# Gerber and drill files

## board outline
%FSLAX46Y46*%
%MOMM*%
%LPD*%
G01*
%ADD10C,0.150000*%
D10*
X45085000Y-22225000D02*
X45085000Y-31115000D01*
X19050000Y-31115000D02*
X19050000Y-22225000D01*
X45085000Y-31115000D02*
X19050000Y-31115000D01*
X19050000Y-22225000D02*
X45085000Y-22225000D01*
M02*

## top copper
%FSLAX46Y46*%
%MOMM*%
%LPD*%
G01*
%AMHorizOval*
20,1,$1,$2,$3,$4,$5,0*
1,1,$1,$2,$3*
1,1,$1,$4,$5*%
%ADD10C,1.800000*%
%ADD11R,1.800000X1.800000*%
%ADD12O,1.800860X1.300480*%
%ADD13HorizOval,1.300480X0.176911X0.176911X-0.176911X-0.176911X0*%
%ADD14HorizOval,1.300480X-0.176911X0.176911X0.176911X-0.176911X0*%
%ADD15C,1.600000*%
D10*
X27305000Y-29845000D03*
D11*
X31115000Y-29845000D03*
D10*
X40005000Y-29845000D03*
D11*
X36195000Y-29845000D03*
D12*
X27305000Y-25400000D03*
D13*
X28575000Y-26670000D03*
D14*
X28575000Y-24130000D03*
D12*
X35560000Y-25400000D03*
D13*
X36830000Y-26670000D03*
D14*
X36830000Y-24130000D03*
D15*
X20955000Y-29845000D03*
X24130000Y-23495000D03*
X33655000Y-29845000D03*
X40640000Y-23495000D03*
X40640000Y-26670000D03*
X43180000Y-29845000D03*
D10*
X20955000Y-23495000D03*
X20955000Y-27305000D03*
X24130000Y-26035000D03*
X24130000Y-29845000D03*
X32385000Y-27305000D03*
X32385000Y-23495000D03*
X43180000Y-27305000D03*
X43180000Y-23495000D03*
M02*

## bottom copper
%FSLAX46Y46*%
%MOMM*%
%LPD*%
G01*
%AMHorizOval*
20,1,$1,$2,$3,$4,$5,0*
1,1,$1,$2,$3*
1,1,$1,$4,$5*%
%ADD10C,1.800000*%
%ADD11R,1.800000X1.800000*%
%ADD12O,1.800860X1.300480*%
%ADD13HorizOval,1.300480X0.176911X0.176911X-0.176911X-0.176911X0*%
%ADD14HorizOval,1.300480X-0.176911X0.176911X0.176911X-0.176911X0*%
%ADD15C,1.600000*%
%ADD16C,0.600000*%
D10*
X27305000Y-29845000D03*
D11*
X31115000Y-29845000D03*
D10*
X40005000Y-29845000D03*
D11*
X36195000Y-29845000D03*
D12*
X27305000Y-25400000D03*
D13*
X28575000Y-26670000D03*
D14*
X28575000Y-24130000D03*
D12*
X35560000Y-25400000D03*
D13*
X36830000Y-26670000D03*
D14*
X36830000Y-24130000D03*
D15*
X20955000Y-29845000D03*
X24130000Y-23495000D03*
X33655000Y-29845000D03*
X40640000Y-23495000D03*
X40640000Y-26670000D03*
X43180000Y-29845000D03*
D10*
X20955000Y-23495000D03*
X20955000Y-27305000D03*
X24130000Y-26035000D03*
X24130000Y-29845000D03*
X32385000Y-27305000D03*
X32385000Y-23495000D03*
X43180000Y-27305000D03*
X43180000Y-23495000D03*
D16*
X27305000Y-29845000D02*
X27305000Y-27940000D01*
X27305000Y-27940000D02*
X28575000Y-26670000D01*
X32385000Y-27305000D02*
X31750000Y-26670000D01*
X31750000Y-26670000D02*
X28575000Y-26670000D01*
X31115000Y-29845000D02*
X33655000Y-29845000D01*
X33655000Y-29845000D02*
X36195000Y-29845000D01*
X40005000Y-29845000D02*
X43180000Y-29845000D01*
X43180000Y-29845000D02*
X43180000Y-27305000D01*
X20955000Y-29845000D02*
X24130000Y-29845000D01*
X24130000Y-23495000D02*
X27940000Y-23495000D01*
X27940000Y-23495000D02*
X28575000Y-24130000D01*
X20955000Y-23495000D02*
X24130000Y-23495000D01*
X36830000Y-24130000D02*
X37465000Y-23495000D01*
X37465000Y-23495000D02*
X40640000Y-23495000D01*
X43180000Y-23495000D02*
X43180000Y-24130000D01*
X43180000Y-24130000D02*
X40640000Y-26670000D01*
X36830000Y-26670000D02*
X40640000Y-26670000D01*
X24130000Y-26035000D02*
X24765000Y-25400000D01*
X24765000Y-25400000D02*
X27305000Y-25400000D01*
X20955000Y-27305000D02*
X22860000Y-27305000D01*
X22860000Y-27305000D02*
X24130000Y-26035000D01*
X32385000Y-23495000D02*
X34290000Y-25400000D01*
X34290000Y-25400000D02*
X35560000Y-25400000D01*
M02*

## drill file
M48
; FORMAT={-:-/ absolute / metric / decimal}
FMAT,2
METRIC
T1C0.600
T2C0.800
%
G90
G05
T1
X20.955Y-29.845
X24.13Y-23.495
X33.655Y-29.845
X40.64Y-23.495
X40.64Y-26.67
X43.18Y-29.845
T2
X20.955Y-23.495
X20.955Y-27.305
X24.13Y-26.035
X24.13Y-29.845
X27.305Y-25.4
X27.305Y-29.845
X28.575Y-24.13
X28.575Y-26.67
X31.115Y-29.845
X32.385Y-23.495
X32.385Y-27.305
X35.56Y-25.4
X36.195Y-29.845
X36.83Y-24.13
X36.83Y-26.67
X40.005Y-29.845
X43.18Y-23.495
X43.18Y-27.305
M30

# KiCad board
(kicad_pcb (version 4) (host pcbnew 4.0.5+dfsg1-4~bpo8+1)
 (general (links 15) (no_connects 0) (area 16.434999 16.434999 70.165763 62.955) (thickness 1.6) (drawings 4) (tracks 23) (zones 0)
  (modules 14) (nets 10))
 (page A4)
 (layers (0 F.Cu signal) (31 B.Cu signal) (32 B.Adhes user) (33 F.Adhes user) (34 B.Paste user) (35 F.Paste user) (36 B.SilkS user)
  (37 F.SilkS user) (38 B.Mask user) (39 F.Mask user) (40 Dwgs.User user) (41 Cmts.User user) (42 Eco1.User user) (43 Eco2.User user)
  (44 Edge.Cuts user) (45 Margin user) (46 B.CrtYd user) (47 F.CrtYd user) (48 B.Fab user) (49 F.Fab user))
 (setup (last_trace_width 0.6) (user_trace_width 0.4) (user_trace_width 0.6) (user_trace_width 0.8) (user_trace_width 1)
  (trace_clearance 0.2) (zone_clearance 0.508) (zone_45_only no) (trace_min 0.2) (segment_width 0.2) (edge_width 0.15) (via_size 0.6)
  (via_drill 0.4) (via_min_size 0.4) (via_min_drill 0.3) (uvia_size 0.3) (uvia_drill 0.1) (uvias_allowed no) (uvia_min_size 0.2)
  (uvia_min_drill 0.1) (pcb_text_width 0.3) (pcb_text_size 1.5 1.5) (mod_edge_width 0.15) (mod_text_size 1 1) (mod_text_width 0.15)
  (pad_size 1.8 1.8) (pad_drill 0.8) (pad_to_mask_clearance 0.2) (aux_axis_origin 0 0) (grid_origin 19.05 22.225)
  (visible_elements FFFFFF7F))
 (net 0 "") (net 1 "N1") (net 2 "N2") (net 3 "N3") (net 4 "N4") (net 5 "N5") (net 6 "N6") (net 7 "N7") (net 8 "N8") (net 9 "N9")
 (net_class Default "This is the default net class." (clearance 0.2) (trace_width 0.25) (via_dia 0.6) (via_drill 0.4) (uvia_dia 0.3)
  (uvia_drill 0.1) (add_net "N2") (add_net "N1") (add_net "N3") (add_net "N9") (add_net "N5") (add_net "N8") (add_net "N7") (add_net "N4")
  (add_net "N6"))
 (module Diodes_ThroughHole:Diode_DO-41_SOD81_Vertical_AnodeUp (layer F.Cu) (at 31.115 29.845 180)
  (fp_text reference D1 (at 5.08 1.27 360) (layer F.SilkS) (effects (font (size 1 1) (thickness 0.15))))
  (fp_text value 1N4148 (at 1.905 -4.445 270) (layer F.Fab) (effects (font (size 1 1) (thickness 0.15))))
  (pad 2 thru_hole circle (at 3.81 0 180) (size 1.8 1.8) (drill 0.8) (layers *.Cu *.Mask) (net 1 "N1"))
  (pad 1 thru_hole rect (at 0 0 180) (size 1.8 1.8) (drill 0.8) (layers *.Cu *.Mask) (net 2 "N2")))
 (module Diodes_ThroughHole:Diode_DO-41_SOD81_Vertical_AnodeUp (layer F.Cu) (at 36.195 29.845)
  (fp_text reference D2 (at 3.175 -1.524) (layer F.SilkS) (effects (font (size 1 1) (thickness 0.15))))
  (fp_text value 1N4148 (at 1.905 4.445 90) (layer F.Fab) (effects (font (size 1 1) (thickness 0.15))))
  (pad 2 thru_hole circle (at 3.81 0) (size 1.8 1.8) (drill 0.8) (layers *.Cu *.Mask) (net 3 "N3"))
  (pad 1 thru_hole rect (at 0 0) (size 1.8 1.8) (drill 0.8) (layers *.Cu *.Mask) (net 2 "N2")))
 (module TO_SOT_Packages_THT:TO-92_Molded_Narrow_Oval (layer F.Cu) (at 28.575 26.67 90)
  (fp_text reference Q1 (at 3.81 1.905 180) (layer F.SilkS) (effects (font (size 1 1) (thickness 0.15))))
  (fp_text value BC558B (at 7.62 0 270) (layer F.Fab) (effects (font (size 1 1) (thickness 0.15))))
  (pad 2 thru_hole oval (at 1.27 -1.27 180) (size 1.80086 1.30048) (drill 0.8) (layers *.Cu *.Mask) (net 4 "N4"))
  (pad 1 thru_hole oval (at 0 0 135) (size 1.30048 1.80086) (drill 0.8) (layers *.Cu *.Mask) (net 1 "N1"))
  (pad 3 thru_hole oval (at 2.54 0 135) (size 1.80086 1.30048) (drill 0.8) (layers *.Cu *.Mask) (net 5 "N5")))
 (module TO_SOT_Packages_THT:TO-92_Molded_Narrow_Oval (layer F.Cu) (at 36.83 26.67 90)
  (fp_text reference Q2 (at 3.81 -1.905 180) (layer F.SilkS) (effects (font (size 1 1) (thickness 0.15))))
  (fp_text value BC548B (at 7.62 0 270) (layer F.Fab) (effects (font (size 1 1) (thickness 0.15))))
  (pad 2 thru_hole oval (at 1.27 -1.27 180) (size 1.80086 1.30048) (drill 0.8) (layers *.Cu *.Mask) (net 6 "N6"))
  (pad 1 thru_hole oval (at 0 0 135) (size 1.30048 1.80086) (drill 0.8) (layers *.Cu *.Mask) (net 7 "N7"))
  (pad 3 thru_hole oval (at 2.54 0 135) (size 1.80086 1.30048) (drill 0.8) (layers *.Cu *.Mask) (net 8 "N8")))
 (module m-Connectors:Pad (layer F.Cu) (at 20.955 29.845)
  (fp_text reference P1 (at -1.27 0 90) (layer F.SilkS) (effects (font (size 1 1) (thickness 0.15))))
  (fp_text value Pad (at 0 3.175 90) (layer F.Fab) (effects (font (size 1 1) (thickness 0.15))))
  (pad 1 thru_hole circle (at 0 0) (size 1.6 1.6) (drill 0.6) (layers *.Cu *.Mask) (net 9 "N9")))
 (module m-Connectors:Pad (layer F.Cu) (at 24.13 23.495)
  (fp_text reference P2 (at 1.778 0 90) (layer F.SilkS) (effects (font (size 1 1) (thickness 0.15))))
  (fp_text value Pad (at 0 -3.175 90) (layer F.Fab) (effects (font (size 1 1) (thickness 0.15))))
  (pad 1 thru_hole circle (at 0 0) (size 1.6 1.6) (drill 0.6) (layers *.Cu *.Mask) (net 5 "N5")))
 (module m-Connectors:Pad (layer F.Cu) (at 33.655 29.845)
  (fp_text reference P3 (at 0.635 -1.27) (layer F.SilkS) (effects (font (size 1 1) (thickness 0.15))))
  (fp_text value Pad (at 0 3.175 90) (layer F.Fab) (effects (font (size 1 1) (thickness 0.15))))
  (pad 1 thru_hole circle (at 0 0) (size 1.6 1.6) (drill 0.6) (layers *.Cu *.Mask) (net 2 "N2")))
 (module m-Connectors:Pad (layer F.Cu) (at 40.64 23.495)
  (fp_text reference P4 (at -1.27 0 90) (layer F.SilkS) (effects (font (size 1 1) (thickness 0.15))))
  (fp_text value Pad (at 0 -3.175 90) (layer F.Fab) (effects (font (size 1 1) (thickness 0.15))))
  (pad 1 thru_hole circle (at 0 0) (size 1.6 1.6) (drill 0.6) (layers *.Cu *.Mask) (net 8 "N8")))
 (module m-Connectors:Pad (layer F.Cu) (at 40.64 26.67)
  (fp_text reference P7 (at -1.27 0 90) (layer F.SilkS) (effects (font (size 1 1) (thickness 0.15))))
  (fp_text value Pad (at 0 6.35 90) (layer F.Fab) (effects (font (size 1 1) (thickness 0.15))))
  (pad 1 thru_hole circle (at 0 0) (size 1.6 1.6) (drill 0.6) (layers *.Cu *.Mask) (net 7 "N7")))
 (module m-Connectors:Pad (layer F.Cu) (at 43.18 29.845)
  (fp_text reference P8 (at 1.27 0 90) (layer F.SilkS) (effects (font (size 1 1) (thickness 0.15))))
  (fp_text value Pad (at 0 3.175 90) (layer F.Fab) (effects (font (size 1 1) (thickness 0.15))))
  (pad 1 thru_hole circle (at 0 0) (size 1.6 1.6) (drill 0.6) (layers *.Cu *.Mask) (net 3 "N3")))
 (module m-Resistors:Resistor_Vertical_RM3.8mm (layer F.Cu) (at 20.955 26.035 270)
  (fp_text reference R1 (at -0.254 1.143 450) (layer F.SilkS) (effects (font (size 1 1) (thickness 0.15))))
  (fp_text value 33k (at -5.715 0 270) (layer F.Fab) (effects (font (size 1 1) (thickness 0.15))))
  (pad 1 thru_hole circle (at -2.54 0 270) (size 1.8 1.8) (drill 0.8) (layers *.Cu *.SilkS *.Mask) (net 5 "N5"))
  (pad 2 thru_hole circle (at 1.27 0 270) (size 1.8 1.8) (drill 0.8) (layers *.Cu *.SilkS *.Mask) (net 4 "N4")))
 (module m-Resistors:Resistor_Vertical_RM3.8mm (layer F.Cu) (at 24.13 28.575 270)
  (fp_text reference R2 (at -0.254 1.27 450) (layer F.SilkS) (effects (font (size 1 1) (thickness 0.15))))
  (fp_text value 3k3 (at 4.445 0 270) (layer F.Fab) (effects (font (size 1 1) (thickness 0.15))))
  (pad 1 thru_hole circle (at -2.54 0 270) (size 1.8 1.8) (drill 0.8) (layers *.Cu *.SilkS *.Mask) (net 4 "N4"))
  (pad 2 thru_hole circle (at 1.27 0 270) (size 1.8 1.8) (drill 0.8) (layers *.Cu *.SilkS *.Mask) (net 9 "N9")))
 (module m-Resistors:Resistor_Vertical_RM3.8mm (layer F.Cu) (at 32.385 24.765 90)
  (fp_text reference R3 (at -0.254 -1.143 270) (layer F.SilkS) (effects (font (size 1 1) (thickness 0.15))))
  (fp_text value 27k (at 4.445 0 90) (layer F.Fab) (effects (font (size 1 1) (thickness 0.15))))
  (pad 1 thru_hole circle (at -2.54 0 90) (size 1.8 1.8) (drill 0.8) (layers *.Cu *.SilkS *.Mask) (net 1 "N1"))
  (pad 2 thru_hole circle (at 1.27 0 90) (size 1.8 1.8) (drill 0.8) (layers *.Cu *.SilkS *.Mask) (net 6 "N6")))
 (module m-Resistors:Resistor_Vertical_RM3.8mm (layer F.Cu) (at 43.18 24.765 90)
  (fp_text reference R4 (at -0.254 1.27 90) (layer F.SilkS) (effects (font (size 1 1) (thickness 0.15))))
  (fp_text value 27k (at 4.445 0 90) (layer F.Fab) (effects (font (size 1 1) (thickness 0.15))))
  (pad 1 thru_hole circle (at -2.54 0 90) (size 1.8 1.8) (drill 0.8) (layers *.Cu *.SilkS *.Mask) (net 3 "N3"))
  (pad 2 thru_hole circle (at 1.27 0 90) (size 1.8 1.8) (drill 0.8) (layers *.Cu *.SilkS *.Mask) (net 7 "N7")))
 (gr_line (start 45.085 22.225) (end 45.085 31.115) (angle 90) (layer Edge.Cuts) (width 0.15))
 (gr_line (start 19.05 31.115) (end 19.05 22.225) (angle 90) (layer Edge.Cuts) (width 0.15))
 (gr_line (start 45.085 31.115) (end 19.05 31.115) (angle 90) (layer Edge.Cuts) (width 0.15))
 (gr_line (start 19.05 22.225) (end 45.085 22.225) (angle 90) (layer Edge.Cuts) (width 0.15))
 (segment (start 27.305 29.845) (end 27.305 27.94) (width 0.6) (layer B.Cu) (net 1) (status 400000))
 (segment (start 27.305 27.94) (end 28.575 26.67) (width 0.6) (layer B.Cu) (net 1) (status 800000))
 (segment (start 32.385 27.305) (end 31.75 26.67) (width 0.6) (layer B.Cu) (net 1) (status C00000))
 (segment (start 31.75 26.67) (end 28.575 26.67) (width 0.6) (layer B.Cu) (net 1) (status C00000))
 (segment (start 31.115 29.845) (end 33.655 29.845) (width 0.6) (layer B.Cu) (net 2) (status C00000))
 (segment (start 33.655 29.845) (end 36.195 29.845) (width 0.6) (layer B.Cu) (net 2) (status C00000))
 (segment (start 40.005 29.845) (end 43.18 29.845) (width 0.6) (layer B.Cu) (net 3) (status C00000))
 (segment (start 43.18 29.845) (end 43.18 27.305) (width 0.6) (layer B.Cu) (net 3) (status C00000))
 (segment (start 20.955 29.845) (end 24.13 29.845) (width 0.6) (layer B.Cu) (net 9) (status C00000))
 (segment (start 24.13 23.495) (end 27.94 23.495) (width 0.6) (layer B.Cu) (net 5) (status C00000))
 (segment (start 27.94 23.495) (end 28.575 24.13) (width 0.6) (layer B.Cu) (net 5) (status C00000))
 (segment (start 20.955 23.495) (end 24.13 23.495) (width 0.6) (layer B.Cu) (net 5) (status C00000))
 (segment (start 36.83 24.13) (end 37.465 23.495) (width 0.6) (layer B.Cu) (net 8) (status 400000))
 (segment (start 37.465 23.495) (end 40.64 23.495) (width 0.6) (layer B.Cu) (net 8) (status 800000))
 (segment (start 43.18 23.495) (end 43.18 24.13) (width 0.6) (layer B.Cu) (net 7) (status C00000))
 (segment (start 43.18 24.13) (end 40.64 26.67) (width 0.6) (layer B.Cu) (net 7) (status C00000))
 (segment (start 36.83 26.67) (end 40.64 26.67) (width 0.6) (layer B.Cu) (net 7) (status C00000))
 (segment (start 24.13 26.035) (end 24.765 25.4) (width 0.6) (layer B.Cu) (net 4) (status C00000))
 (segment (start 24.765 25.4) (end 27.305 25.4) (width 0.6) (layer B.Cu) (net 4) (status C00000))
 (segment (start 20.955 27.305) (end 22.86 27.305) (width 0.6) (layer B.Cu) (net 4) (status 400000))
 (segment (start 22.86 27.305) (end 24.13 26.035) (width 0.6) (layer B.Cu) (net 4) (status 800000))
 (segment (start 32.385 23.495) (end 34.29 25.4) (width 0.6) (layer B.Cu) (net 6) (status 400000))
 (segment (start 34.29 25.4) (end 35.56 25.4) (width 0.6) (layer B.Cu) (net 6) (status 800000)))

